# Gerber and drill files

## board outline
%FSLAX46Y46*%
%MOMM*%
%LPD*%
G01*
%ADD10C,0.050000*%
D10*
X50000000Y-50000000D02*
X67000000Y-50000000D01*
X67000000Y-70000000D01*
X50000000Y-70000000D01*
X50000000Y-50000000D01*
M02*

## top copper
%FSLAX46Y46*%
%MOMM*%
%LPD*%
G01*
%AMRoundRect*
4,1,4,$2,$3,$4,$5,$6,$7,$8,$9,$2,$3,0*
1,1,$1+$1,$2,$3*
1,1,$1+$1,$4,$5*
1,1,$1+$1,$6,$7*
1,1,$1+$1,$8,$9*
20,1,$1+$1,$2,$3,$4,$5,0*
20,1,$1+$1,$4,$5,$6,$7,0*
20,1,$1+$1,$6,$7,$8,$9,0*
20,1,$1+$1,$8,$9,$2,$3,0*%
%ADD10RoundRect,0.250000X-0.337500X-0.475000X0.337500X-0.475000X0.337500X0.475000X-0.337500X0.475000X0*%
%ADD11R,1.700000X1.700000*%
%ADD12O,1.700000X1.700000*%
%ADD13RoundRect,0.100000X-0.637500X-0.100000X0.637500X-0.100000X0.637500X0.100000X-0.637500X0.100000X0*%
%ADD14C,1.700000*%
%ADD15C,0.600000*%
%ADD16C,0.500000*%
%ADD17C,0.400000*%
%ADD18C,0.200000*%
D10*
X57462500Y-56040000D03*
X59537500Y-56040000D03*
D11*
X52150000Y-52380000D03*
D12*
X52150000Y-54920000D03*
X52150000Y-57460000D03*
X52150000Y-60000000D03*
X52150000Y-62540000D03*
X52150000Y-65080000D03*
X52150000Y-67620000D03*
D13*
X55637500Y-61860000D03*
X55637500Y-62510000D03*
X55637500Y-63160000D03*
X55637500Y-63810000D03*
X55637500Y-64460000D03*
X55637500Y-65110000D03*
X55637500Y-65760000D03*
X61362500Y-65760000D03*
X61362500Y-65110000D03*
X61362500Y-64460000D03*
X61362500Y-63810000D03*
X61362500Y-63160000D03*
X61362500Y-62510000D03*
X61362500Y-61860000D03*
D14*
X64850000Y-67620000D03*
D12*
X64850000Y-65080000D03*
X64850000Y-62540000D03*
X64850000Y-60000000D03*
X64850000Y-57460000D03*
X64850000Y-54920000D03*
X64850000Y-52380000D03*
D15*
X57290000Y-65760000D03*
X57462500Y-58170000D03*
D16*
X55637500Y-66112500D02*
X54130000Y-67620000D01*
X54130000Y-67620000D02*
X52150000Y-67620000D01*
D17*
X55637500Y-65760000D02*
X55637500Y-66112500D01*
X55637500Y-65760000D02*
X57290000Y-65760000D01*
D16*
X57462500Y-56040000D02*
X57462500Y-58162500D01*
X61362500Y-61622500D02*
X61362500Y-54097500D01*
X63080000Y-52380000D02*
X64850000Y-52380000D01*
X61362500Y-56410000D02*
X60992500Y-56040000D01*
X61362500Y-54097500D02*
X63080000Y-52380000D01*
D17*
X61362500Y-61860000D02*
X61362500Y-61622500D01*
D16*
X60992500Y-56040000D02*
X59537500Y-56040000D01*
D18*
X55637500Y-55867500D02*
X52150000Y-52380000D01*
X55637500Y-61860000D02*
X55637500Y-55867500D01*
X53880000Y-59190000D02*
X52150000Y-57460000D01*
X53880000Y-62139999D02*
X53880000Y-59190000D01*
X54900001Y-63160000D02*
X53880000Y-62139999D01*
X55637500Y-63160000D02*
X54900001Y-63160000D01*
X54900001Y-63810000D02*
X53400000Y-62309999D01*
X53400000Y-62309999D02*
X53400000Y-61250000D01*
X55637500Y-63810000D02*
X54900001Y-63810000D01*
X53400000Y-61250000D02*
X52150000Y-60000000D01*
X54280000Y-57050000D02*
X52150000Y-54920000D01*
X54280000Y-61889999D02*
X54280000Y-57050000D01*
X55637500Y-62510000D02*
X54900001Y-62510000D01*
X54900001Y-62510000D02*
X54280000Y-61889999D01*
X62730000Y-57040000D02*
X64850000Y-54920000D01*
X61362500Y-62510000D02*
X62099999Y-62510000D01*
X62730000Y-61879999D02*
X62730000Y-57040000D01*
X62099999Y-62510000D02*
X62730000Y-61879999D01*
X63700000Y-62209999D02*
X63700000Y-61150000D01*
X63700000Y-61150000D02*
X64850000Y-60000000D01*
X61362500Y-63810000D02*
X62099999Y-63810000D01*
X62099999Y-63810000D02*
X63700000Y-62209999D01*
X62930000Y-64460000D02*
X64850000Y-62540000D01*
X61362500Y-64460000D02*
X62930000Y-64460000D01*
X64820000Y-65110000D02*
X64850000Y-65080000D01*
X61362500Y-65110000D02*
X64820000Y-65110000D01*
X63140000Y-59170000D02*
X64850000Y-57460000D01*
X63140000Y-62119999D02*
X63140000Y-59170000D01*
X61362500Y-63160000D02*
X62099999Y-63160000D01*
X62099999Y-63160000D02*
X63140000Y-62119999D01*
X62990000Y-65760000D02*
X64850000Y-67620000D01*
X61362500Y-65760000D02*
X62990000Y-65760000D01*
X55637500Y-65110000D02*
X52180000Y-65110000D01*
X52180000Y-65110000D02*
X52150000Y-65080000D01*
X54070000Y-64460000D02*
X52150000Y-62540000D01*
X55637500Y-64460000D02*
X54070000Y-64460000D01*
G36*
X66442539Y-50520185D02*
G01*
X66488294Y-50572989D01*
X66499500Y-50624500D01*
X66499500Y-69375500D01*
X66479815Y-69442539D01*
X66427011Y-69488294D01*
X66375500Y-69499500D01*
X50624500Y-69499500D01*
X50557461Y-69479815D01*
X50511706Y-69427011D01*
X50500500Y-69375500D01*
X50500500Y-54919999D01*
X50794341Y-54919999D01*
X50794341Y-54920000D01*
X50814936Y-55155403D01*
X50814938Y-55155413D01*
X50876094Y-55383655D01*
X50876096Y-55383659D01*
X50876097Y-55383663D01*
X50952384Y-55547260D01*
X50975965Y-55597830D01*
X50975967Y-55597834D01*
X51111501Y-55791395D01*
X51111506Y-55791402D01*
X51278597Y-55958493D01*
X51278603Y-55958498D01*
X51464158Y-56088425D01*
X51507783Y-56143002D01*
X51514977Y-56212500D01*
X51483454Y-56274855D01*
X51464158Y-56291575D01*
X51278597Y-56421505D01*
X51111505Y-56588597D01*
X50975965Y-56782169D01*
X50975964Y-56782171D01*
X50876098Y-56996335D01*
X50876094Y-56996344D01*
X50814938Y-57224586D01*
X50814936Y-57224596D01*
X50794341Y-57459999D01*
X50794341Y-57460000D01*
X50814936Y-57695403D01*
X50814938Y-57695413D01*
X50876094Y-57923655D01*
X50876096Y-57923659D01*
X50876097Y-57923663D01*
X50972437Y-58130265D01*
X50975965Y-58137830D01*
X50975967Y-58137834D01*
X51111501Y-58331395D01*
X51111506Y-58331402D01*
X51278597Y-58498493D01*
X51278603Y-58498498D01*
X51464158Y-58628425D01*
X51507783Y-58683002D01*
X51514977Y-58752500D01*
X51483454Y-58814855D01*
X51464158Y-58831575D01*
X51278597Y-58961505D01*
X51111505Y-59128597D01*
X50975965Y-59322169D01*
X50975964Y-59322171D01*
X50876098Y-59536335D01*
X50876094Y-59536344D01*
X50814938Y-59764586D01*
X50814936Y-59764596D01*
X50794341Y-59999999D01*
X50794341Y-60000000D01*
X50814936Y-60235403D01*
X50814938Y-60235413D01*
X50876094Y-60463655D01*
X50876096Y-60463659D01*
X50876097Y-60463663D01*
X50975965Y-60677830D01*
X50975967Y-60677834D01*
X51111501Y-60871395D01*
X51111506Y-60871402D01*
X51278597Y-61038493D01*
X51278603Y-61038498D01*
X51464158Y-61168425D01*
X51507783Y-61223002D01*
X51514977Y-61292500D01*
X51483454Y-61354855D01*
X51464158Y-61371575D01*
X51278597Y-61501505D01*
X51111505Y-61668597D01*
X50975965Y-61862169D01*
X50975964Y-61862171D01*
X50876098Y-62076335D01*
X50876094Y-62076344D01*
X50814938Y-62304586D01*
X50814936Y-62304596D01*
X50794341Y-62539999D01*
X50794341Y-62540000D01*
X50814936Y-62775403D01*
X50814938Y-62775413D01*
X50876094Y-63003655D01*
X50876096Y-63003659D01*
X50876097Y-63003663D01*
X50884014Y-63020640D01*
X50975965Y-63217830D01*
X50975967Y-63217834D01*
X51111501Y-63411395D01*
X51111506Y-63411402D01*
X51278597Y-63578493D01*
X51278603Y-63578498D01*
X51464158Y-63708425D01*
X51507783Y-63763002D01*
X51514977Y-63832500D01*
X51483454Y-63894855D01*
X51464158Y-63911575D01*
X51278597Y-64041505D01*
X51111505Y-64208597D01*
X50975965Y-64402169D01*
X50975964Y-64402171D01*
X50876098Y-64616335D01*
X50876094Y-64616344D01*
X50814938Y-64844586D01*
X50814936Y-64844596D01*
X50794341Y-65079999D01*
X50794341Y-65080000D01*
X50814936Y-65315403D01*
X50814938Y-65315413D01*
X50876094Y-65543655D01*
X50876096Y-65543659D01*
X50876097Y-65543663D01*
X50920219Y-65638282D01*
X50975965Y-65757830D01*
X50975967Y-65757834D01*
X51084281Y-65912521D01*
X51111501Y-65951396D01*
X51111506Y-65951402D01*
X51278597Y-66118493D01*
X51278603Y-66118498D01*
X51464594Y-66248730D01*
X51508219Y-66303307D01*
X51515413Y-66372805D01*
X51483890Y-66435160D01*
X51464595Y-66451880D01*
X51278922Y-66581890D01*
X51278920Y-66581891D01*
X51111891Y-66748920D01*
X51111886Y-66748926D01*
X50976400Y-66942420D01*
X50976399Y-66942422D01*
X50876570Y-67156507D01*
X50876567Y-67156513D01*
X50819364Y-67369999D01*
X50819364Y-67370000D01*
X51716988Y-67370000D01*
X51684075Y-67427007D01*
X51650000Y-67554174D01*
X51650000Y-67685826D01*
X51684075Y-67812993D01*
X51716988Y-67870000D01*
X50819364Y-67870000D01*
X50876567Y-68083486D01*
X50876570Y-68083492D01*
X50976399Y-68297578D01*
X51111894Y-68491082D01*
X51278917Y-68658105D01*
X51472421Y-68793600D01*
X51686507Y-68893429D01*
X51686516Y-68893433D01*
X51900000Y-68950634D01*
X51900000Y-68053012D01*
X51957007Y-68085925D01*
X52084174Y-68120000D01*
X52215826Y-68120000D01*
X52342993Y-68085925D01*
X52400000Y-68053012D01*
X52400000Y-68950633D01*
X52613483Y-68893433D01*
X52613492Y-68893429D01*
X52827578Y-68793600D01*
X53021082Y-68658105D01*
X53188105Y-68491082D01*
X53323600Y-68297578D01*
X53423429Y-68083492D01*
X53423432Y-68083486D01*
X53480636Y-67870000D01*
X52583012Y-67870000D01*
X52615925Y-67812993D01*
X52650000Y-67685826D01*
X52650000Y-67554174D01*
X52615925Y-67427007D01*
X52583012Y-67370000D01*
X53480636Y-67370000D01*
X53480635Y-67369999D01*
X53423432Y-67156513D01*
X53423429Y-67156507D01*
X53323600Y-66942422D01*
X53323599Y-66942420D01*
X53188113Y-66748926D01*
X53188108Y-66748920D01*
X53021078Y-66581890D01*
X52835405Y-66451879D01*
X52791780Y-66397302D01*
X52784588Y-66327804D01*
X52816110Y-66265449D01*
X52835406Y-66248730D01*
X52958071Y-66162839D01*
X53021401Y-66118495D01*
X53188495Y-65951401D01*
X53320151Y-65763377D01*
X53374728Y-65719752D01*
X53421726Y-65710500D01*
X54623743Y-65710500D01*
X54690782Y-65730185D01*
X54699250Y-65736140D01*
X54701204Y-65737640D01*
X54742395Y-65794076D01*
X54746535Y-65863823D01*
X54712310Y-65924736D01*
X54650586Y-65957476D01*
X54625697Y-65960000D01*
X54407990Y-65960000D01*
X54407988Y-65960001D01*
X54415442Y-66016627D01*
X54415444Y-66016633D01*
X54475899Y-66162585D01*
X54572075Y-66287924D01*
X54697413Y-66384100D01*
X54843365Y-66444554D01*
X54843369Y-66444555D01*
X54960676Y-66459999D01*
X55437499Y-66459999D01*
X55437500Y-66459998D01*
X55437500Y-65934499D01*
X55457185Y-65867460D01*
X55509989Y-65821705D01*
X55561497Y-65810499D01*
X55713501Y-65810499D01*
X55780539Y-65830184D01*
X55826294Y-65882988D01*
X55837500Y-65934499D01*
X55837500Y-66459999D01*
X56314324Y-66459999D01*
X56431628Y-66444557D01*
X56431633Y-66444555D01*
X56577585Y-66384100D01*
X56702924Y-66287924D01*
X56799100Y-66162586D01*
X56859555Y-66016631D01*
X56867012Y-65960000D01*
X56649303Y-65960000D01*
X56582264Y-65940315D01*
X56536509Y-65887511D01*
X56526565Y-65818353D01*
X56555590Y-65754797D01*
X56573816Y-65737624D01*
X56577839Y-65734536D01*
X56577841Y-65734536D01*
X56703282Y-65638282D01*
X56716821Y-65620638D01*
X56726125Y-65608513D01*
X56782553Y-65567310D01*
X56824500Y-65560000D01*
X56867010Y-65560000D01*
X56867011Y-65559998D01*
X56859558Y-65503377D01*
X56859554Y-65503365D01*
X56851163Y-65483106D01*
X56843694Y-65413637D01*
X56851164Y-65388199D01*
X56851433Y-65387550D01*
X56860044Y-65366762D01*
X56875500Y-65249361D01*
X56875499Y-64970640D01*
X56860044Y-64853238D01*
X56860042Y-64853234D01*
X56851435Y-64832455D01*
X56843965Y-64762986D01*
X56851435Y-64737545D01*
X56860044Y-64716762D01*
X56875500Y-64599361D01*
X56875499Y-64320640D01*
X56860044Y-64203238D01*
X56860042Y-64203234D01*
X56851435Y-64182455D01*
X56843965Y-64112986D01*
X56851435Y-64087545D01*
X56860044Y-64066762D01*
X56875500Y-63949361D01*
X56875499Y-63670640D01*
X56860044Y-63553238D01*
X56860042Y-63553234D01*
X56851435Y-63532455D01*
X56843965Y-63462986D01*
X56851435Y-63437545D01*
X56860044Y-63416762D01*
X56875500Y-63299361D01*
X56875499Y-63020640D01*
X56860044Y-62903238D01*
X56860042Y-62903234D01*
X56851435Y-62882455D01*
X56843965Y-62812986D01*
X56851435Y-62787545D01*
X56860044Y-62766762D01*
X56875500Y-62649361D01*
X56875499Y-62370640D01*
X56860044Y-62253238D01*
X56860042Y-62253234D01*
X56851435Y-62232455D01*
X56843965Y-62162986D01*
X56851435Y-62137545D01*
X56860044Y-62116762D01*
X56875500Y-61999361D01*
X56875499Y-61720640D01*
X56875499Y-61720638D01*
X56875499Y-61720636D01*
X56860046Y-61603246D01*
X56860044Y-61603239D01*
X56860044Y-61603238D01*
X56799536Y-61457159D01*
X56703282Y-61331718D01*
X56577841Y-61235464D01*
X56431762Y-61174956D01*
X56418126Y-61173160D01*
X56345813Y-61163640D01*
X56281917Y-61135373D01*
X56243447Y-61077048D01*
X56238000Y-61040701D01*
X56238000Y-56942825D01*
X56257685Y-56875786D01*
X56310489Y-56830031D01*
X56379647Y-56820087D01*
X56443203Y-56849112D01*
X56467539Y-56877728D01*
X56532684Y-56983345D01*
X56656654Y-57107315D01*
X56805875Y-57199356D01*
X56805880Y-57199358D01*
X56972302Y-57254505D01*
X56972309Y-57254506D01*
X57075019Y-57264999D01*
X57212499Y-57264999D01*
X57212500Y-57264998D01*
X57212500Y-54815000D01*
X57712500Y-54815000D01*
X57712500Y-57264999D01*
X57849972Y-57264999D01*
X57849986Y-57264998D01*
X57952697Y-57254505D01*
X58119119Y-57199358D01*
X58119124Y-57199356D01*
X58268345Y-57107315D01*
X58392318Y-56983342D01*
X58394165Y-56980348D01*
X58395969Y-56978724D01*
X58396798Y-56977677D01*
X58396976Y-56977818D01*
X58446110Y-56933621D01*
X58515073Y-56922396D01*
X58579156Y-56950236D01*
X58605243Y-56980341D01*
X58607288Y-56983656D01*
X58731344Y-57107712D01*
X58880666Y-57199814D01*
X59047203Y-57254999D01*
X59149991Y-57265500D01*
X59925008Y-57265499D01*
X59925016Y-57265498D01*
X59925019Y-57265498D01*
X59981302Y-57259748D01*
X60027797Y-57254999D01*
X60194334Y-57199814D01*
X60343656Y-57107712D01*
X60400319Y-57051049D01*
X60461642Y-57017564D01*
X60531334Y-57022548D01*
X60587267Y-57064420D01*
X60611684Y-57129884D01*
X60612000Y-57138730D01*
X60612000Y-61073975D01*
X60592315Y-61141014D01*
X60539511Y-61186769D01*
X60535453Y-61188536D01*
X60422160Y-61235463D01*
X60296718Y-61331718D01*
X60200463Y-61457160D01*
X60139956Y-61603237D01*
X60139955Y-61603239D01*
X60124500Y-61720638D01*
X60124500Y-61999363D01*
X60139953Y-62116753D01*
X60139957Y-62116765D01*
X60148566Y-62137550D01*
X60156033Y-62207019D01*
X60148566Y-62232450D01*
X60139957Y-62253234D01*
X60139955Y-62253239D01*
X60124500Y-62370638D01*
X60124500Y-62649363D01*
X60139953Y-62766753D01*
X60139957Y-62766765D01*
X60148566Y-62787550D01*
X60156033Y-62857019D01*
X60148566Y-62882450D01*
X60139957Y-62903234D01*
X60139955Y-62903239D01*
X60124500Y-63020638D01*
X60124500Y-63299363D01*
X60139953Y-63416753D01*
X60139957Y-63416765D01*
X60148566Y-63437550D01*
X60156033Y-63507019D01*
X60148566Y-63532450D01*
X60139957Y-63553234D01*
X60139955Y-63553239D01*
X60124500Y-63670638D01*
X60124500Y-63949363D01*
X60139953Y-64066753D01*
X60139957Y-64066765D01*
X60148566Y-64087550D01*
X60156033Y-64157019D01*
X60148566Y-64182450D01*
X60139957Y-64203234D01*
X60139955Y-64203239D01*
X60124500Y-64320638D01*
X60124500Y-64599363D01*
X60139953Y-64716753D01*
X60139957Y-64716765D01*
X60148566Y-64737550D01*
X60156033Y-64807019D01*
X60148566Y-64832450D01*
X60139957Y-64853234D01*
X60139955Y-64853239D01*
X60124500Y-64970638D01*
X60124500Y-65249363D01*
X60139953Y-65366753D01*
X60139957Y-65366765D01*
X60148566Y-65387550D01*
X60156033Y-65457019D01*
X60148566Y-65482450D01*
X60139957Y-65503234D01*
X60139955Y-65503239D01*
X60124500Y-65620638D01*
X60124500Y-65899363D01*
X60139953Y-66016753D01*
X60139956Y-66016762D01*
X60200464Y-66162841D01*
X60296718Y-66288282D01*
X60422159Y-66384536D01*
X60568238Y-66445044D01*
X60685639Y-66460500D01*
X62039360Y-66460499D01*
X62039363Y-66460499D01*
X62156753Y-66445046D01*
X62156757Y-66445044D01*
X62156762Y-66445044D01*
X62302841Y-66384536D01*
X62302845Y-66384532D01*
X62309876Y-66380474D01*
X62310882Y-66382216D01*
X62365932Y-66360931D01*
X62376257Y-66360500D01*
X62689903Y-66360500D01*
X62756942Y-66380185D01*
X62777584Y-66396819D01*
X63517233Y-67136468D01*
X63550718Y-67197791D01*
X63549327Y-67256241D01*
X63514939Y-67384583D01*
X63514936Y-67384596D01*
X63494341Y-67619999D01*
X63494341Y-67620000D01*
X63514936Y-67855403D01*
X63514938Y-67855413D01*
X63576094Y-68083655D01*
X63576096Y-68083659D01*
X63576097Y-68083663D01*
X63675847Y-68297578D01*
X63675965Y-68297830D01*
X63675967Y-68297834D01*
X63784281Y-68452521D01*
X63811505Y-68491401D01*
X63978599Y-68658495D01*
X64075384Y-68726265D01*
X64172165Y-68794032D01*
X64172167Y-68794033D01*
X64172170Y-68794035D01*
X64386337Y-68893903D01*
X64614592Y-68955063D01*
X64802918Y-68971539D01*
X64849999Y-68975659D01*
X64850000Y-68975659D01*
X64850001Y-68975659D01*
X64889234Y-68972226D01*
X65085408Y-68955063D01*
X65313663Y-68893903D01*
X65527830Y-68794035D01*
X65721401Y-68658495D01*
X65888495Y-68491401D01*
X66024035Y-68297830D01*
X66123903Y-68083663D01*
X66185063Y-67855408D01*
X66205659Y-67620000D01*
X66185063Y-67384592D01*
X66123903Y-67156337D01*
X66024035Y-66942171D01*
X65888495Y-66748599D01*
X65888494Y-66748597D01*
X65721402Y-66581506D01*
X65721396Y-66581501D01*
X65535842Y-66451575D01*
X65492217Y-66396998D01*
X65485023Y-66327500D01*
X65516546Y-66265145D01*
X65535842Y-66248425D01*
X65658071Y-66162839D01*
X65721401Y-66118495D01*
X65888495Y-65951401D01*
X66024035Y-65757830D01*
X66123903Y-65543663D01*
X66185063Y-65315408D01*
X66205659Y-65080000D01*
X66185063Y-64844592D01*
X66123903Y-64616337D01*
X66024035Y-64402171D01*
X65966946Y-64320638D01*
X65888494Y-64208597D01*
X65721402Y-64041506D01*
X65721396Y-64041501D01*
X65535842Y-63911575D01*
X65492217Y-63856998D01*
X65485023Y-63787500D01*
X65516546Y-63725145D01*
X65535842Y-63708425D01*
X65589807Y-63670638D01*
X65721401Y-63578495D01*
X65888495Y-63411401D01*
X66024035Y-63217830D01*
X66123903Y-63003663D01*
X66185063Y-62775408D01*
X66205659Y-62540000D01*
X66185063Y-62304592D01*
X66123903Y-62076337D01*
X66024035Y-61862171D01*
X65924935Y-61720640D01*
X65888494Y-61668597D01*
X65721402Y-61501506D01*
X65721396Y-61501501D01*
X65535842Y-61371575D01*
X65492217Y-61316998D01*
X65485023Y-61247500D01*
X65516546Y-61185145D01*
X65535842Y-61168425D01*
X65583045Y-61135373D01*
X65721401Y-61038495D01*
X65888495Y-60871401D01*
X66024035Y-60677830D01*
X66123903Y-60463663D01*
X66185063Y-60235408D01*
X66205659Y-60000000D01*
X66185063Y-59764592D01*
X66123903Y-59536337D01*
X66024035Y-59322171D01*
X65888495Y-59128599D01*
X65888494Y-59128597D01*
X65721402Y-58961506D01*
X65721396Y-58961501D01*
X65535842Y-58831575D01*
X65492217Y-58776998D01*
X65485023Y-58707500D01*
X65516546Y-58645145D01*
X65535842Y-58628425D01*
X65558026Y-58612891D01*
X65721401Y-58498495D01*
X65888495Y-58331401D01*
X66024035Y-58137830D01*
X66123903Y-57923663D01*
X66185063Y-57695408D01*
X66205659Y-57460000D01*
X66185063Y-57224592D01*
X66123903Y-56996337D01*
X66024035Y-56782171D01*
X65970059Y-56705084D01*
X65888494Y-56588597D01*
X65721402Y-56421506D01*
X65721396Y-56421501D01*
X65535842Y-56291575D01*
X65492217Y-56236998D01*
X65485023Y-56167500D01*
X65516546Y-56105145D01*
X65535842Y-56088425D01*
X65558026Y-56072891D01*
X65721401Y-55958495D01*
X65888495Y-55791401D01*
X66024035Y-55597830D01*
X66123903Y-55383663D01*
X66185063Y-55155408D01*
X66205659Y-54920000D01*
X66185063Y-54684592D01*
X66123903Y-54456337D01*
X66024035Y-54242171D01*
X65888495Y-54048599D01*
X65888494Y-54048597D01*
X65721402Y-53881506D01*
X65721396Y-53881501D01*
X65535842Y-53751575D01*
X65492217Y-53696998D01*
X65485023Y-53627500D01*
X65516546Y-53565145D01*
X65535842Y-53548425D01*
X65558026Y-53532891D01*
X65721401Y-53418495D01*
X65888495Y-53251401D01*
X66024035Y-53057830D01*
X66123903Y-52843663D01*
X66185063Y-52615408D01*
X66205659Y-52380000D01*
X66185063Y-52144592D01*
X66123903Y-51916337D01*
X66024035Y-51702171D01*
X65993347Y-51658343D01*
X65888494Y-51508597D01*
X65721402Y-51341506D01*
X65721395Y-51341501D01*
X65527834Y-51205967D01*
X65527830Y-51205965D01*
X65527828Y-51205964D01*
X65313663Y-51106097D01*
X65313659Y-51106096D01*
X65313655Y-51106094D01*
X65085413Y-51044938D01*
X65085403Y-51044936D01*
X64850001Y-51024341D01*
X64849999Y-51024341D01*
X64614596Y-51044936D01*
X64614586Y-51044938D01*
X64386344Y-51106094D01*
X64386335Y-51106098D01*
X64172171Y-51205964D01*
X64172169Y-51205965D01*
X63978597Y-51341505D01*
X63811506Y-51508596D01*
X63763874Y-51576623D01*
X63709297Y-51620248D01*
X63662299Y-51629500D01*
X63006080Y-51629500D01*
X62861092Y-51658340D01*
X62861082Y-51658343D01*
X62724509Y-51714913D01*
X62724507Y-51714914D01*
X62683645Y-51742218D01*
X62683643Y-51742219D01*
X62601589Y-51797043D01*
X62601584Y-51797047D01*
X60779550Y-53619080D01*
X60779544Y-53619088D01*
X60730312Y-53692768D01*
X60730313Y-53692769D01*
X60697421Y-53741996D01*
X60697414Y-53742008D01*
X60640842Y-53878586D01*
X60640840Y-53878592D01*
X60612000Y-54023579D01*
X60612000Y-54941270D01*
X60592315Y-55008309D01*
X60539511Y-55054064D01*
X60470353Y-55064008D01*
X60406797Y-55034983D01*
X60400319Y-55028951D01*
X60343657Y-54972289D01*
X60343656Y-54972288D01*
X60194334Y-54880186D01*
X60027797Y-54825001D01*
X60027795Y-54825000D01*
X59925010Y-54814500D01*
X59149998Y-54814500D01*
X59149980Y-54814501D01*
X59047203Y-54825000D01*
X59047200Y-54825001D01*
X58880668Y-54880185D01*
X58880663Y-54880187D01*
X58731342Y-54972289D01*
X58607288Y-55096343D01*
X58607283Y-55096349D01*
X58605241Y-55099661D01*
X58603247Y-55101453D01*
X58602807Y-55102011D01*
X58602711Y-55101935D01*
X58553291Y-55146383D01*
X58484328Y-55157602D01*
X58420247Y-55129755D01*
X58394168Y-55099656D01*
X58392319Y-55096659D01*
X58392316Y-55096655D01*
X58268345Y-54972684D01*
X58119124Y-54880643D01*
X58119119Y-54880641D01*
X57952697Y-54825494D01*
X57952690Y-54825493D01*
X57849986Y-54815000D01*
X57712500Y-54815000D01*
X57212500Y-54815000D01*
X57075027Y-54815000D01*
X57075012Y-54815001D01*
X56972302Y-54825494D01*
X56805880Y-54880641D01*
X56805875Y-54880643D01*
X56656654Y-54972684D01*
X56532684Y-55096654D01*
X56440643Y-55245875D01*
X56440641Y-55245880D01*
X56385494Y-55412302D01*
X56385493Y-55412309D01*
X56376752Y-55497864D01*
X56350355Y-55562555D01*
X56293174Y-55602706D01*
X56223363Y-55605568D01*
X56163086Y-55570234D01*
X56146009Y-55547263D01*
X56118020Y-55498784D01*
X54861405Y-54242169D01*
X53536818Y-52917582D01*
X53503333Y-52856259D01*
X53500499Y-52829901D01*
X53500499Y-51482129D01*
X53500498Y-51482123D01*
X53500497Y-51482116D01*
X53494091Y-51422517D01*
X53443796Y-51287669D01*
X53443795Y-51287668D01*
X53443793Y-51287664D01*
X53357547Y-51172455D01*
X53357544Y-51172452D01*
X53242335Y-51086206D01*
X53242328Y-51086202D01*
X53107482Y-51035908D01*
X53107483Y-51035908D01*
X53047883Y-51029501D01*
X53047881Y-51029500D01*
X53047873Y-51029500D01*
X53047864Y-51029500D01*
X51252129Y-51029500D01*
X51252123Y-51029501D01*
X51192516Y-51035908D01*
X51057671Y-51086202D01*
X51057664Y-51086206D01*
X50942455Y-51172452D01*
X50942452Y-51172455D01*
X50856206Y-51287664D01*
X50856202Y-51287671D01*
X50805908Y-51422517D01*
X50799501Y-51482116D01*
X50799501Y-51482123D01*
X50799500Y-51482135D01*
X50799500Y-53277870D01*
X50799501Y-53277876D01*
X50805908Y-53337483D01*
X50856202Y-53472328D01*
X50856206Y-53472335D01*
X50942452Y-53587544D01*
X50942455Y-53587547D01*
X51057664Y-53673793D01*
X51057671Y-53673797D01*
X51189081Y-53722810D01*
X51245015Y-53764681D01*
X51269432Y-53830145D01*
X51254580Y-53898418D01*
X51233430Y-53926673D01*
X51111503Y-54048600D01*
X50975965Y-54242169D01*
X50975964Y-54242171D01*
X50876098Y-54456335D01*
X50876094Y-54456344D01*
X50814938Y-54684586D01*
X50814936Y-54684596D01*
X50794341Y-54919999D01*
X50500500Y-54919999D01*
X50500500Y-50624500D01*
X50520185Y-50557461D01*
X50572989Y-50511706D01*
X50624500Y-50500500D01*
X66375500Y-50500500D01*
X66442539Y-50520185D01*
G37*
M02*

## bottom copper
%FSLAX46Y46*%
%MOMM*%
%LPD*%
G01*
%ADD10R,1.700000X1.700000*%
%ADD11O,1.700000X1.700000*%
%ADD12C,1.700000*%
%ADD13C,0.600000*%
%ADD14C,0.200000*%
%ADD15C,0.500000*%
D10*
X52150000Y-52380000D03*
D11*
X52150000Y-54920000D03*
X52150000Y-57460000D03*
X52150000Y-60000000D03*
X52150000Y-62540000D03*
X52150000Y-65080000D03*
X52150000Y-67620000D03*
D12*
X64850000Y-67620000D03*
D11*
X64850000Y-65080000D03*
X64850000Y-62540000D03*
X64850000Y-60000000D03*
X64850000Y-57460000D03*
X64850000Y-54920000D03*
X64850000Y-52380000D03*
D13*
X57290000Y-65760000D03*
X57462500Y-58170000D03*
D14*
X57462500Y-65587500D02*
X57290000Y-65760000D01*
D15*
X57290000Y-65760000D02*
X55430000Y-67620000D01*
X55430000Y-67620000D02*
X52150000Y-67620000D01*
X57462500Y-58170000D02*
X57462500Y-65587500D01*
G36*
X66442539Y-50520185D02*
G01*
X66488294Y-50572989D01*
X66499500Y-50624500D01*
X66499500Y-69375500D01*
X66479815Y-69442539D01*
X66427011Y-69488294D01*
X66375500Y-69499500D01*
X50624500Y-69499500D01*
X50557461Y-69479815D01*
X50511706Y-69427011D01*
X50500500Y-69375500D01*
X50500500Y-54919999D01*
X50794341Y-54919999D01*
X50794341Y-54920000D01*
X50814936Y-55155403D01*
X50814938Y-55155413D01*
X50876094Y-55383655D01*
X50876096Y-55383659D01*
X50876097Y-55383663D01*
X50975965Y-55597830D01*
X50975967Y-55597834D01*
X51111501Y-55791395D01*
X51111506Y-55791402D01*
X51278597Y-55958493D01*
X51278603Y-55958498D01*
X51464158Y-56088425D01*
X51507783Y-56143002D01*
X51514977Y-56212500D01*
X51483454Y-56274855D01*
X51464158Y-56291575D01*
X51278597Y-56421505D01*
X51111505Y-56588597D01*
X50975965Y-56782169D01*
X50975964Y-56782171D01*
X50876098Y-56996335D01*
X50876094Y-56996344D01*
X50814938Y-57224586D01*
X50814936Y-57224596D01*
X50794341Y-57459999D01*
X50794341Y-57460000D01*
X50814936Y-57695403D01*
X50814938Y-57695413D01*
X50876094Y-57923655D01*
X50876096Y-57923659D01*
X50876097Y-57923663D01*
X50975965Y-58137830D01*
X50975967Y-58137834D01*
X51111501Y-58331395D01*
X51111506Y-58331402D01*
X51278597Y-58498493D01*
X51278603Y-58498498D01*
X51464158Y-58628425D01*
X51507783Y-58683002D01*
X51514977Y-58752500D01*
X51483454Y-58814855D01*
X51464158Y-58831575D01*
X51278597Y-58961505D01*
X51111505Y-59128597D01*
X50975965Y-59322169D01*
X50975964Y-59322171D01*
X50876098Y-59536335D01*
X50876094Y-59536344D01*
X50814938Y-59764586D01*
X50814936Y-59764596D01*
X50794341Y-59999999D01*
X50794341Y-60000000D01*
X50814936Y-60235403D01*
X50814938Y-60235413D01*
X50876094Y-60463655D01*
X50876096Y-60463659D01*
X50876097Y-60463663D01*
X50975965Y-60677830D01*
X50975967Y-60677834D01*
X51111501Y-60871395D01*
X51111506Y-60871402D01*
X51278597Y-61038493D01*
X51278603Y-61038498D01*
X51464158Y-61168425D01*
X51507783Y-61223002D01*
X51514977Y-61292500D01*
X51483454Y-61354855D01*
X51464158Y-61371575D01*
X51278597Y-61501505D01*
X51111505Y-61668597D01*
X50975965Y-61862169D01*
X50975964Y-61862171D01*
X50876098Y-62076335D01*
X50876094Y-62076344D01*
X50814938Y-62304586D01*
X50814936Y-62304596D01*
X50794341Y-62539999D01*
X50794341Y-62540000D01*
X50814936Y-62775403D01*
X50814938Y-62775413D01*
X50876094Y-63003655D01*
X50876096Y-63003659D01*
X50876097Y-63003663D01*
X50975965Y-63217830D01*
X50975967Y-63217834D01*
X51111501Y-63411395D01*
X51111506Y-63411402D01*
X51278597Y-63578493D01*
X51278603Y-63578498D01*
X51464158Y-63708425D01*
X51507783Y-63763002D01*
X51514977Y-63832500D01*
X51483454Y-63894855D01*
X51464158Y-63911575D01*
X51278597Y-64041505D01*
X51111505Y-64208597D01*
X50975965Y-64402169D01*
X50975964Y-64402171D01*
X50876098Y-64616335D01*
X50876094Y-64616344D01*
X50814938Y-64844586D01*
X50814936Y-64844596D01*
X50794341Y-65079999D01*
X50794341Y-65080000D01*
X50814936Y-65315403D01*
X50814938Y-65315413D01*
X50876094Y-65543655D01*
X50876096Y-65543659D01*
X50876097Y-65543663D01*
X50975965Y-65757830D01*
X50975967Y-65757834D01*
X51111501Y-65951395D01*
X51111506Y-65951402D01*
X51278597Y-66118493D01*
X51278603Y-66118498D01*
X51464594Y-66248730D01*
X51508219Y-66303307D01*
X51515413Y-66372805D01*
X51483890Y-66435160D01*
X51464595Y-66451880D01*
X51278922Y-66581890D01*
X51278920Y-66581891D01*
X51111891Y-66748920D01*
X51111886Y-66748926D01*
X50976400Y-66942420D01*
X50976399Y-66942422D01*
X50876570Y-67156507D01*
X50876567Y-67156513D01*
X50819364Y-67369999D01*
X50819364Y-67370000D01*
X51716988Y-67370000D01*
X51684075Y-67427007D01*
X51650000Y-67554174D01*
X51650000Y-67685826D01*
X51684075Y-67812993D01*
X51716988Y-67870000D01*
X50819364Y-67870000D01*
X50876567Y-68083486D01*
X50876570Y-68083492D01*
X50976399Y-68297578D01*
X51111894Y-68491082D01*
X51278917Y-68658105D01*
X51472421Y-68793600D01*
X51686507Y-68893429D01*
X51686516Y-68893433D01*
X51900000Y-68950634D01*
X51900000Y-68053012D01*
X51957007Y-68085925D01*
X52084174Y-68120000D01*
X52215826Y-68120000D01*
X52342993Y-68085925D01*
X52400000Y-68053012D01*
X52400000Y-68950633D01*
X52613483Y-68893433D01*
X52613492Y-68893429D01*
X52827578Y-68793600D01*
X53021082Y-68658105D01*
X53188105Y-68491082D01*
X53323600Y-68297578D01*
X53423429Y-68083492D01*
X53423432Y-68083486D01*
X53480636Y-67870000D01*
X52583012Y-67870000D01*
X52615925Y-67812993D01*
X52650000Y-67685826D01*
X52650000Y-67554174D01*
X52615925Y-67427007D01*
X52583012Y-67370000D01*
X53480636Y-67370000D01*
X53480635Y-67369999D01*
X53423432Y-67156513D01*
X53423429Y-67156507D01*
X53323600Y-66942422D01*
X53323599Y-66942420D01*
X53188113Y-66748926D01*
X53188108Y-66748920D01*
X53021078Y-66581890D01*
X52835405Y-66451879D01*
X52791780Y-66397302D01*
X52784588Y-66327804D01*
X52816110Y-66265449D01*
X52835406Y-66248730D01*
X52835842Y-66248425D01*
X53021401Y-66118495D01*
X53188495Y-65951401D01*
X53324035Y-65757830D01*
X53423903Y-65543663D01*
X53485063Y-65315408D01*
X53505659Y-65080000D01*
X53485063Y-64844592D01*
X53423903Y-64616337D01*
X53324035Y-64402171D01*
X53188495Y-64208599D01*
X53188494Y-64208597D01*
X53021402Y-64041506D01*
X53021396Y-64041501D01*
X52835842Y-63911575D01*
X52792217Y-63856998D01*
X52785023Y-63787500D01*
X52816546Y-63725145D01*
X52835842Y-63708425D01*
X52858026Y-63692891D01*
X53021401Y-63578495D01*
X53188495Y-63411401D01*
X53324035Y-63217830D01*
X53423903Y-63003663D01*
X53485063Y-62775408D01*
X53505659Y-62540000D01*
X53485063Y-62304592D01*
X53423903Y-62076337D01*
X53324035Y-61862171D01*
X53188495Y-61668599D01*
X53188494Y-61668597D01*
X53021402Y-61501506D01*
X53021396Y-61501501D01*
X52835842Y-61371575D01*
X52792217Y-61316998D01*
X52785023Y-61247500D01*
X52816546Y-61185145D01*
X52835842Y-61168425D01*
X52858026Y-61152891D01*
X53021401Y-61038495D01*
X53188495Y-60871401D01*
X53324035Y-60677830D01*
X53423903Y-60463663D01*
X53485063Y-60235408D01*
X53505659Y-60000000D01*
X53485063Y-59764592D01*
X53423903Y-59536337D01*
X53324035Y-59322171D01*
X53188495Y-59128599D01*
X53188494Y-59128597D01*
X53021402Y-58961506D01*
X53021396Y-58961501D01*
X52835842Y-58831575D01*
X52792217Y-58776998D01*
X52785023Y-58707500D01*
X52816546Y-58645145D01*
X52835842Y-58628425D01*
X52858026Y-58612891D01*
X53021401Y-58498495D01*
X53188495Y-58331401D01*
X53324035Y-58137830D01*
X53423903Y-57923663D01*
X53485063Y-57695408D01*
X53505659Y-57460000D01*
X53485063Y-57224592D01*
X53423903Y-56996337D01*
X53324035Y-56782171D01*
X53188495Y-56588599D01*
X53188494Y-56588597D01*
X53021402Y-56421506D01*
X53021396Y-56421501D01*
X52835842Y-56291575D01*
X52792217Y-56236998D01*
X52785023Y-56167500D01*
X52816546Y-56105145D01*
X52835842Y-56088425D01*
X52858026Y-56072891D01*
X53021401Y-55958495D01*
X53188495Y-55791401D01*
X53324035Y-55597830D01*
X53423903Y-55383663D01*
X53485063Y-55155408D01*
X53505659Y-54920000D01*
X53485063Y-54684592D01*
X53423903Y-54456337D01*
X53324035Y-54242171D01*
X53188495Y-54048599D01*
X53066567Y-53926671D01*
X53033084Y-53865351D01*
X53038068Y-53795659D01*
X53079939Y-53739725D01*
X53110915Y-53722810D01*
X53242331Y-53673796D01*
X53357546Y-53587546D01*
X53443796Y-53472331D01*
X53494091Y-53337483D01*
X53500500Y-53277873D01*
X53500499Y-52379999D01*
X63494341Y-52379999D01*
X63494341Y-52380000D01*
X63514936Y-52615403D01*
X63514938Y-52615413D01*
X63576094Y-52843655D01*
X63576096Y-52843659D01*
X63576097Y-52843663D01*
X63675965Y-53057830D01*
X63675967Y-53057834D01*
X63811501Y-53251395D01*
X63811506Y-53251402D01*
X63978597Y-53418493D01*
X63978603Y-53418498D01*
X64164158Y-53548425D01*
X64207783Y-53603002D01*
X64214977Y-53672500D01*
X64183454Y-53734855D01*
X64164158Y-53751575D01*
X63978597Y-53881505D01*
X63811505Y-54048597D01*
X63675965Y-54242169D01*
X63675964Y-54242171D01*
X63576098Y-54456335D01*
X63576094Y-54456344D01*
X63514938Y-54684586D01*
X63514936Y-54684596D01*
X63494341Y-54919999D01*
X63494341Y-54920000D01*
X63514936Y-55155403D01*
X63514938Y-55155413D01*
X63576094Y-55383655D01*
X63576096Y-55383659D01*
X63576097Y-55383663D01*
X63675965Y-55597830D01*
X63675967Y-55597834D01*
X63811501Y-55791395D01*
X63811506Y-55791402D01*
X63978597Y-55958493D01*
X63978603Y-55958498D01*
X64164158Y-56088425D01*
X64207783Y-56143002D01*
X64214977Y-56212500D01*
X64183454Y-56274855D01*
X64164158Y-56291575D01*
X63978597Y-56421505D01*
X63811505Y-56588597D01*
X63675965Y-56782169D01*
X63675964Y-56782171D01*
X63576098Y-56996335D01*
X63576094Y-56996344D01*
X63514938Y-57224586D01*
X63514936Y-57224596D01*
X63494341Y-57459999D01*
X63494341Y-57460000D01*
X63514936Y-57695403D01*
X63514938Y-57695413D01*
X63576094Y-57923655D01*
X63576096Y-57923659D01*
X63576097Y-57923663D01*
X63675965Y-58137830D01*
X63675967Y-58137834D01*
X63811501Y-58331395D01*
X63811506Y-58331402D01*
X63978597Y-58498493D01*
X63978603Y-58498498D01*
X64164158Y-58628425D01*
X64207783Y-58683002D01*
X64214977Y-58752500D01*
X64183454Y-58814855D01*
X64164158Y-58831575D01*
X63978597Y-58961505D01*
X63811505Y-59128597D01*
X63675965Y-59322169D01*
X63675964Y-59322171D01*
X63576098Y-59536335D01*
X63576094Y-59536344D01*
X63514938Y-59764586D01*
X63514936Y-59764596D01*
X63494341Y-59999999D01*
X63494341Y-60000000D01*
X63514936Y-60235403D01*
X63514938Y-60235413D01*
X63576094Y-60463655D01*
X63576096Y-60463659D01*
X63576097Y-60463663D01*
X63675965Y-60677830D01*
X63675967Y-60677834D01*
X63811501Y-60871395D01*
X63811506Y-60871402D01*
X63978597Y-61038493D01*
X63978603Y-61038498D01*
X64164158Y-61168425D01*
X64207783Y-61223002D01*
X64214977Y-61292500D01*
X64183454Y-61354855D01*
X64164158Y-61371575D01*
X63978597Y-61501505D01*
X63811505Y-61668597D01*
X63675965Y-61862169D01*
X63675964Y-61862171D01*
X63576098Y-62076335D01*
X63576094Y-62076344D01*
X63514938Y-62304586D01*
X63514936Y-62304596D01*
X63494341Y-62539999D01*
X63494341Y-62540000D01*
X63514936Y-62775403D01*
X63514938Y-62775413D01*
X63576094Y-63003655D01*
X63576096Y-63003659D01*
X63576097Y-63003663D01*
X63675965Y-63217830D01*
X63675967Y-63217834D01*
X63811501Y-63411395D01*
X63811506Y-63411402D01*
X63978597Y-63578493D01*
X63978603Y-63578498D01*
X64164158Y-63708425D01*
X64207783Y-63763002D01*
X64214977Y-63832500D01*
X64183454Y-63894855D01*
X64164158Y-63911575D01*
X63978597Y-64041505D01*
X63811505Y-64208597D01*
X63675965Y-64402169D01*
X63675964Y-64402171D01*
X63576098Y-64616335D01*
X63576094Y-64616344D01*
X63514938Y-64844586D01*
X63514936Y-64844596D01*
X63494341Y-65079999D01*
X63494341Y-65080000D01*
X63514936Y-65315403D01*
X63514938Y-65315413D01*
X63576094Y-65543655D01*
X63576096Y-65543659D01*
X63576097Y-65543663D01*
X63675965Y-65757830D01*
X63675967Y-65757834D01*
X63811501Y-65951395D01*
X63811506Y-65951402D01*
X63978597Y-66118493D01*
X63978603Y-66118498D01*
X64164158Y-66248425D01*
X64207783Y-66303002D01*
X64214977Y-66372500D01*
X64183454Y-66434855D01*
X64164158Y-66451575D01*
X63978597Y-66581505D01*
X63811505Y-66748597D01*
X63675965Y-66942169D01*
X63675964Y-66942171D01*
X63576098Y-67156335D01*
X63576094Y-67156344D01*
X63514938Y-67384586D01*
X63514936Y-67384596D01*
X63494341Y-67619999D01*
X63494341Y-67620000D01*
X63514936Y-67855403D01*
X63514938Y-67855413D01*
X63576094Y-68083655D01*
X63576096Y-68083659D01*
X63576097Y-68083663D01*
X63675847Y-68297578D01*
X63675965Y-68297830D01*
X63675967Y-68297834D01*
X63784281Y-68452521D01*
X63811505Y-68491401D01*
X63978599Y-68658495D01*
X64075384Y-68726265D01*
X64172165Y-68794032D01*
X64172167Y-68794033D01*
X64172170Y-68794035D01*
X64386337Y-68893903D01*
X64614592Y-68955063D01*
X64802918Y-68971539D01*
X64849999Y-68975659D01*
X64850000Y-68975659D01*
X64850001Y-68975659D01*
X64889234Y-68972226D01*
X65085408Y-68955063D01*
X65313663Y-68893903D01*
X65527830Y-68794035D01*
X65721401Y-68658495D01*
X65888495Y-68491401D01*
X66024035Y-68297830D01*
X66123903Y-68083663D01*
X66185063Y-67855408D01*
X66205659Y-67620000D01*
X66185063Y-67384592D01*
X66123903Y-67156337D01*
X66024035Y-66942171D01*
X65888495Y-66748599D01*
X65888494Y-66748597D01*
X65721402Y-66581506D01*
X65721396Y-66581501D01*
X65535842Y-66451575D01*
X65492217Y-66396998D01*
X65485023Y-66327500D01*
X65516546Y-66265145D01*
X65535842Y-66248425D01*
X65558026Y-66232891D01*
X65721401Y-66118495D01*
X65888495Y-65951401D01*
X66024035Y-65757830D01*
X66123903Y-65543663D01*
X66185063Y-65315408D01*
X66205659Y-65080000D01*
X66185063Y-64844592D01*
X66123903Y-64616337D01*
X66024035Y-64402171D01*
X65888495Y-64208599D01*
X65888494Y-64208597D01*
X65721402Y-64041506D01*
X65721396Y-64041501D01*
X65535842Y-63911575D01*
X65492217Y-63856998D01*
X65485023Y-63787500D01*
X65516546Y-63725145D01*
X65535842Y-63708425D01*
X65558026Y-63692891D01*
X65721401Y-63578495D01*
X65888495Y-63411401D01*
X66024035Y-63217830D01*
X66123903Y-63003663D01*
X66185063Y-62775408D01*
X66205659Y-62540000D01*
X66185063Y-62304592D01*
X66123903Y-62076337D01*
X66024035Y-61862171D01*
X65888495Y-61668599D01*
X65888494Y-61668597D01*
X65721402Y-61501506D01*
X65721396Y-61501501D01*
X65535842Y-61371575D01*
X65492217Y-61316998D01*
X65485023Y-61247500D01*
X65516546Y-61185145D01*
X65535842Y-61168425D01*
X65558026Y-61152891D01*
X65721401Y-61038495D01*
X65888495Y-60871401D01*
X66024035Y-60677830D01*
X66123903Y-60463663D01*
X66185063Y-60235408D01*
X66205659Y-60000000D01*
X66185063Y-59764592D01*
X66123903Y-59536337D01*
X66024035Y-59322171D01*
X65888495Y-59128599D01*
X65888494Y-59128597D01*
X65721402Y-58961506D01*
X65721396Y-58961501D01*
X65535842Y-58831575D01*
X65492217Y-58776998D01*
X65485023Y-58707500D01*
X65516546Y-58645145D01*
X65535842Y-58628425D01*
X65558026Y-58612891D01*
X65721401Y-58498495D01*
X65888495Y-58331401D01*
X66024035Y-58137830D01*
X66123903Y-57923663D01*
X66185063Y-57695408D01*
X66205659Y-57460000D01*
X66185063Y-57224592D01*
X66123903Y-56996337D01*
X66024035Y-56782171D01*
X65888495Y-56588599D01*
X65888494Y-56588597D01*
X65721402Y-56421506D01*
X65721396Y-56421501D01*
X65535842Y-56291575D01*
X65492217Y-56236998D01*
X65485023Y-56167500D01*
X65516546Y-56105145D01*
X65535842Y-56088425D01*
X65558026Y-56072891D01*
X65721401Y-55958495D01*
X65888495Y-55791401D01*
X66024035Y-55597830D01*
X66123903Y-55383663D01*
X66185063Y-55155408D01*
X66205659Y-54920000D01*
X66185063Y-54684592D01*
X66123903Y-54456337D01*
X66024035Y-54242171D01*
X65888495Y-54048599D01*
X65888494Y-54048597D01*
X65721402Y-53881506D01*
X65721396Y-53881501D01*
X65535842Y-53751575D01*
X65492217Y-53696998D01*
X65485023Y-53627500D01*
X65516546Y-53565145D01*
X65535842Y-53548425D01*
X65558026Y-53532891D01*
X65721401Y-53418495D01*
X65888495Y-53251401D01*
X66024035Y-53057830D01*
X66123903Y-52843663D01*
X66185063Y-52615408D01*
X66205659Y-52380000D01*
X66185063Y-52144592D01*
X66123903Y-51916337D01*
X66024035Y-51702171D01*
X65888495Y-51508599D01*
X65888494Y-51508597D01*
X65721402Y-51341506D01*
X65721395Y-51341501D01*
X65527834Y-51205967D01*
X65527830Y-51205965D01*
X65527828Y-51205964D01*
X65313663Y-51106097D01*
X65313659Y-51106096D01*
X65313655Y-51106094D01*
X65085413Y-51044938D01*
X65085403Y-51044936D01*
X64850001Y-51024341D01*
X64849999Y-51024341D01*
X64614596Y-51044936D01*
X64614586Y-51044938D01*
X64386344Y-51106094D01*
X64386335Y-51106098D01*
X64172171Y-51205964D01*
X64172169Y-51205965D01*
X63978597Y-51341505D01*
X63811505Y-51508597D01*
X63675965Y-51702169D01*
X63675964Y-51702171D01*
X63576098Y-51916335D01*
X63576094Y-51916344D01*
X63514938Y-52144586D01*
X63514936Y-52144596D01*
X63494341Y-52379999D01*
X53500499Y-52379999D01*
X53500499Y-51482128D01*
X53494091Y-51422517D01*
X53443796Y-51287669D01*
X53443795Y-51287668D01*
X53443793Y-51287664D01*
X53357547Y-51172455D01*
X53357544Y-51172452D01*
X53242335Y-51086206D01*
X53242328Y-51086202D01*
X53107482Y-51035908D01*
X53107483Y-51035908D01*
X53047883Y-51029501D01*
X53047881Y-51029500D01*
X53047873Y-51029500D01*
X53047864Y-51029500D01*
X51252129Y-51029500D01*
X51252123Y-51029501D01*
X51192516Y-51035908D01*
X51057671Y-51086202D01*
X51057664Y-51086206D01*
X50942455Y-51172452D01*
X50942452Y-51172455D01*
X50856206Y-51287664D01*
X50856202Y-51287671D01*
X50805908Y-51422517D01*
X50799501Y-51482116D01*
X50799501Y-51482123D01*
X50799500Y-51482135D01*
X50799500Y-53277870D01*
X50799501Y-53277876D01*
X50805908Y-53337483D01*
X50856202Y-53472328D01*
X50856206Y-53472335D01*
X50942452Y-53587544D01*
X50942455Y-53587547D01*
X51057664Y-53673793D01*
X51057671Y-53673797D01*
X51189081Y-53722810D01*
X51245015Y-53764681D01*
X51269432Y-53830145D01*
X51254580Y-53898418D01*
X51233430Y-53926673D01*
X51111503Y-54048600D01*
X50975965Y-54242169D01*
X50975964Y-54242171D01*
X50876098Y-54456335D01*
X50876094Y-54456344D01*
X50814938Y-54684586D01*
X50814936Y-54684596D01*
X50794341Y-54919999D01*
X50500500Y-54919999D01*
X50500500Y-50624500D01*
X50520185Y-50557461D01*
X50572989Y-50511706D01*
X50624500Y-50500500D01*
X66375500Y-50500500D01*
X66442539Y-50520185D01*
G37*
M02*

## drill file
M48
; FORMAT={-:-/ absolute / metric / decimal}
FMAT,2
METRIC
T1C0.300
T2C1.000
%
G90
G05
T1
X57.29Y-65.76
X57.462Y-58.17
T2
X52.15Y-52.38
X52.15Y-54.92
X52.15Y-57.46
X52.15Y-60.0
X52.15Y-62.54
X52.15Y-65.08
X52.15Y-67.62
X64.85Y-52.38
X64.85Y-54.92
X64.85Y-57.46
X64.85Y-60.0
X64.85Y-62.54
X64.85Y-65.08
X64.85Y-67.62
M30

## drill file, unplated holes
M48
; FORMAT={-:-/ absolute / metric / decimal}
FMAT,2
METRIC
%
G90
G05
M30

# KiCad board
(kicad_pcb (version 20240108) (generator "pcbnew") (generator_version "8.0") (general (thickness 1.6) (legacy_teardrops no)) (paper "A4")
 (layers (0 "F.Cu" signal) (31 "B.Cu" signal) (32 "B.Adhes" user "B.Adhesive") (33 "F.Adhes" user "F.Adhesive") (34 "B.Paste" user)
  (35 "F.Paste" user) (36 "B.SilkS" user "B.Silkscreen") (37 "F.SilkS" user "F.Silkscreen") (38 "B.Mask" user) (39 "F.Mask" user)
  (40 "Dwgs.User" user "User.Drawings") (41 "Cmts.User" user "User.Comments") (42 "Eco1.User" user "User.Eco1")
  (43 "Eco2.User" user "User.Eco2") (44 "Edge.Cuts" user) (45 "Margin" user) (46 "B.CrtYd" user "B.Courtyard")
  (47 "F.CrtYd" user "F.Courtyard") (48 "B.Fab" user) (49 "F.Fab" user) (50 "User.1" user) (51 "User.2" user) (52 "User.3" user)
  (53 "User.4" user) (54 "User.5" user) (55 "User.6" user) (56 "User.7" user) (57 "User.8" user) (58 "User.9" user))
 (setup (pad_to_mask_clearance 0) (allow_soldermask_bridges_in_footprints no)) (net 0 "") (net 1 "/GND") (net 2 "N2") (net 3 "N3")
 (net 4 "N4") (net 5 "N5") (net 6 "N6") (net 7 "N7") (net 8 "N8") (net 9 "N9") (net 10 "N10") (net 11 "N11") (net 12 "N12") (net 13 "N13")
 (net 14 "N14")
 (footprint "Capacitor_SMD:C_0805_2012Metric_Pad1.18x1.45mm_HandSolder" (layer "F.Cu") (at 58.5 56.04)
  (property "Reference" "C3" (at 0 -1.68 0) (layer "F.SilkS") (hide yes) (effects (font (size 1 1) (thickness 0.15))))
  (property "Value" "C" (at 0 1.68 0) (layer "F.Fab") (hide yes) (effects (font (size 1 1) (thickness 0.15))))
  (pad "1" smd roundrect (at -1.0375 0) (size 1.175 1.45) (layers "F.Cu" "F.Paste" "F.Mask") (roundrect_rratio 0.212766) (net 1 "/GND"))
  (pad "2" smd roundrect (at 1.0375 0) (size 1.175 1.45) (layers "F.Cu" "F.Paste" "F.Mask") (roundrect_rratio 0.212766) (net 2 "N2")))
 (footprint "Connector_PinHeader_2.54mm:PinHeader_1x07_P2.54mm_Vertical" (layer "F.Cu") (at 52.15 52.38)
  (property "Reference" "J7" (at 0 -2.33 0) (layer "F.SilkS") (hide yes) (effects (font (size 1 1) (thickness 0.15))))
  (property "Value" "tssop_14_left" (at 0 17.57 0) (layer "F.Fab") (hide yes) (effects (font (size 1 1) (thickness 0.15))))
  (pad "1" thru_hole rect (at 0 0) (size 1.7 1.7) (drill 1) (layers "*.Cu" "*.Mask") (remove_unused_layers no) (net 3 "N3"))
  (pad "2" thru_hole oval (at 0 2.54) (size 1.7 1.7) (drill 1) (layers "*.Cu" "*.Mask") (remove_unused_layers no) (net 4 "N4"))
  (pad "3" thru_hole oval (at 0 5.08) (size 1.7 1.7) (drill 1) (layers "*.Cu" "*.Mask") (remove_unused_layers no) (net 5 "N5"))
  (pad "4" thru_hole oval (at 0 7.62) (size 1.7 1.7) (drill 1) (layers "*.Cu" "*.Mask") (remove_unused_layers no) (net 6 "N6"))
  (pad "5" thru_hole oval (at 0 10.16) (size 1.7 1.7) (drill 1) (layers "*.Cu" "*.Mask") (remove_unused_layers no) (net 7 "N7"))
  (pad "6" thru_hole oval (at 0 12.7) (size 1.7 1.7) (drill 1) (layers "*.Cu" "*.Mask") (remove_unused_layers no) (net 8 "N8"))
  (pad "7" thru_hole oval (at 0 15.24) (size 1.7 1.7) (drill 1) (layers "*.Cu" "*.Mask") (remove_unused_layers no) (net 1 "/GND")))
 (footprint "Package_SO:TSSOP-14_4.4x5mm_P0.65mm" (layer "F.Cu") (at 58.5 63.81)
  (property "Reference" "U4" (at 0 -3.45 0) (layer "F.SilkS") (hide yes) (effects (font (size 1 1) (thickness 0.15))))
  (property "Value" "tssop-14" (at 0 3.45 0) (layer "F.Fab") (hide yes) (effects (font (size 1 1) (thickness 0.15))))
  (pad "1" smd roundrect (at -2.8625 -1.95) (size 1.475 0.4) (layers "F.Cu" "F.Paste" "F.Mask") (roundrect_rratio 0.25) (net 3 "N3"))
  (pad "2" smd roundrect (at -2.8625 -1.3) (size 1.475 0.4) (layers "F.Cu" "F.Paste" "F.Mask") (roundrect_rratio 0.25) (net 4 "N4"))
  (pad "3" smd roundrect (at -2.8625 -0.65) (size 1.475 0.4) (layers "F.Cu" "F.Paste" "F.Mask") (roundrect_rratio 0.25) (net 5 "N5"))
  (pad "4" smd roundrect (at -2.8625 0) (size 1.475 0.4) (layers "F.Cu" "F.Paste" "F.Mask") (roundrect_rratio 0.25) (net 6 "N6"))
  (pad "5" smd roundrect (at -2.8625 0.65) (size 1.475 0.4) (layers "F.Cu" "F.Paste" "F.Mask") (roundrect_rratio 0.25) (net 7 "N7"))
  (pad "6" smd roundrect (at -2.8625 1.3) (size 1.475 0.4) (layers "F.Cu" "F.Paste" "F.Mask") (roundrect_rratio 0.25) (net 8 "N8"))
  (pad "7" smd roundrect (at -2.8625 1.95) (size 1.475 0.4) (layers "F.Cu" "F.Paste" "F.Mask") (roundrect_rratio 0.25) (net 1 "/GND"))
  (pad "8" smd roundrect (at 2.8625 1.95) (size 1.475 0.4) (layers "F.Cu" "F.Paste" "F.Mask") (roundrect_rratio 0.25) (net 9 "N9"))
  (pad "9" smd roundrect (at 2.8625 1.3) (size 1.475 0.4) (layers "F.Cu" "F.Paste" "F.Mask") (roundrect_rratio 0.25) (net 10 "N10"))
  (pad "10" smd roundrect (at 2.8625 0.65) (size 1.475 0.4) (layers "F.Cu" "F.Paste" "F.Mask") (roundrect_rratio 0.25) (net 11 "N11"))
  (pad "11" smd roundrect (at 2.8625 0) (size 1.475 0.4) (layers "F.Cu" "F.Paste" "F.Mask") (roundrect_rratio 0.25) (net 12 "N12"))
  (pad "12" smd roundrect (at 2.8625 -0.65) (size 1.475 0.4) (layers "F.Cu" "F.Paste" "F.Mask") (roundrect_rratio 0.25) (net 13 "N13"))
  (pad "13" smd roundrect (at 2.8625 -1.3) (size 1.475 0.4) (layers "F.Cu" "F.Paste" "F.Mask") (roundrect_rratio 0.25) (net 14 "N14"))
  (pad "14" smd roundrect (at 2.8625 -1.95) (size 1.475 0.4) (layers "F.Cu" "F.Paste" "F.Mask") (roundrect_rratio 0.25) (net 2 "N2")))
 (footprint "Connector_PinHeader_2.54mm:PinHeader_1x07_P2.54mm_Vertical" (layer "F.Cu") (at 64.85 67.62 180)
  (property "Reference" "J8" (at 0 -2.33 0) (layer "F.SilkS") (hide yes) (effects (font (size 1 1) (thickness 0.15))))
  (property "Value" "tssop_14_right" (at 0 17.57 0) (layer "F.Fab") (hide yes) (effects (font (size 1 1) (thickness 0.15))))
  (pad "1" thru_hole circle (at 0 0 180) (size 1.7 1.7) (drill 1) (layers "*.Cu" "*.Mask") (remove_unused_layers no) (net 9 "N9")
   (thermal_bridge_angle 90))
  (pad "2" thru_hole oval (at 0 2.54 180) (size 1.7 1.7) (drill 1) (layers "*.Cu" "*.Mask") (remove_unused_layers no) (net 10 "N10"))
  (pad "3" thru_hole oval (at 0 5.08 180) (size 1.7 1.7) (drill 1) (layers "*.Cu" "*.Mask") (remove_unused_layers no) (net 11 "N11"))
  (pad "4" thru_hole oval (at 0 7.62 180) (size 1.7 1.7) (drill 1) (layers "*.Cu" "*.Mask") (remove_unused_layers no) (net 12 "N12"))
  (pad "5" thru_hole oval (at 0 10.16 180) (size 1.7 1.7) (drill 1) (layers "*.Cu" "*.Mask") (remove_unused_layers no) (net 13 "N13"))
  (pad "6" thru_hole oval (at 0 12.7 180) (size 1.7 1.7) (drill 1) (layers "*.Cu" "*.Mask") (remove_unused_layers no) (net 14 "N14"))
  (pad "7" thru_hole oval (at 0 15.24 180) (size 1.7 1.7) (drill 1) (layers "*.Cu" "*.Mask") (remove_unused_layers no) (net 2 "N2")))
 (gr_rect (start 50 50) (end 67 70) (stroke (width 0.05) (type default)) (fill none) (layer "Edge.Cuts"))
 (segment (start 55.6375 66.1125) (end 54.13 67.62) (width 0.5) (layer "F.Cu") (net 1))
 (segment (start 54.13 67.62) (end 52.15 67.62) (width 0.5) (layer "F.Cu") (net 1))
 (segment (start 55.6375 65.76) (end 55.6375 66.1125) (width 0.4) (layer "F.Cu") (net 1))
 (segment (start 55.6375 65.76) (end 57.29 65.76) (width 0.4) (layer "F.Cu") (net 1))
 (segment (start 57.4625 56.04) (end 57.4625 58.1625) (width 0.5) (layer "F.Cu") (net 1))
 (via (at 57.29 65.76) (size 0.6) (drill 0.3) (layers "F.Cu" "B.Cu") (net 1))
 (via (at 57.4625 58.17) (size 0.6) (drill 0.3) (layers "F.Cu" "B.Cu") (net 1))
 (segment (start 57.4625 65.5875) (end 57.29 65.76) (width 0.2) (layer "B.Cu") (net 1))
 (segment (start 57.29 65.76) (end 55.43 67.62) (width 0.5) (layer "B.Cu") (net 1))
 (segment (start 55.43 67.62) (end 52.15 67.62) (width 0.5) (layer "B.Cu") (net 1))
 (segment (start 57.4625 58.17) (end 57.4625 65.5875) (width 0.5) (layer "B.Cu") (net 1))
 (segment (start 61.3625 61.6225) (end 61.3625 54.0975) (width 0.5) (layer "F.Cu") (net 2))
 (segment (start 63.08 52.38) (end 64.85 52.38) (width 0.5) (layer "F.Cu") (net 2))
 (segment (start 61.3625 56.41) (end 60.9925 56.04) (width 0.5) (layer "F.Cu") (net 2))
 (segment (start 61.3625 54.0975) (end 63.08 52.38) (width 0.5) (layer "F.Cu") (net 2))
 (segment (start 61.3625 61.86) (end 61.3625 61.6225) (width 0.4) (layer "F.Cu") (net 2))
 (segment (start 60.9925 56.04) (end 59.5375 56.04) (width 0.5) (layer "F.Cu") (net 2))
 (segment (start 55.6375 55.8675) (end 52.15 52.38) (width 0.2) (layer "F.Cu") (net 3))
 (segment (start 55.6375 61.86) (end 55.6375 55.8675) (width 0.2) (layer "F.Cu") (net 3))
 (segment (start 53.88 59.19) (end 52.15 57.46) (width 0.2) (layer "F.Cu") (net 5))
 (segment (start 53.88 62.139999) (end 53.88 59.19) (width 0.2) (layer "F.Cu") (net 5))
 (segment (start 54.900001 63.16) (end 53.88 62.139999) (width 0.2) (layer "F.Cu") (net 5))
 (segment (start 55.6375 63.16) (end 54.900001 63.16) (width 0.2) (layer "F.Cu") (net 5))
 (segment (start 54.900001 63.81) (end 53.4 62.309999) (width 0.2) (layer "F.Cu") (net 6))
 (segment (start 53.4 62.309999) (end 53.4 61.25) (width 0.2) (layer "F.Cu") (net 6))
 (segment (start 55.6375 63.81) (end 54.900001 63.81) (width 0.2) (layer "F.Cu") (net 6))
 (segment (start 53.4 61.25) (end 52.15 60) (width 0.2) (layer "F.Cu") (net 6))
 (segment (start 54.28 57.05) (end 52.15 54.92) (width 0.2) (layer "F.Cu") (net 4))
 (segment (start 54.28 61.889999) (end 54.28 57.05) (width 0.2) (layer "F.Cu") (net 4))
 (segment (start 55.6375 62.51) (end 54.900001 62.51) (width 0.2) (layer "F.Cu") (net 4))
 (segment (start 54.900001 62.51) (end 54.28 61.889999) (width 0.2) (layer "F.Cu") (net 4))
 (segment (start 62.73 57.04) (end 64.85 54.92) (width 0.2) (layer "F.Cu") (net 14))
 (segment (start 61.3625 62.51) (end 62.099999 62.51) (width 0.2) (layer "F.Cu") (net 14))
 (segment (start 62.73 61.879999) (end 62.73 57.04) (width 0.2) (layer "F.Cu") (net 14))
 (segment (start 62.099999 62.51) (end 62.73 61.879999) (width 0.2) (layer "F.Cu") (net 14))
 (segment (start 63.7 62.209999) (end 63.7 61.15) (width 0.2) (layer "F.Cu") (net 12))
 (segment (start 63.7 61.15) (end 64.85 60) (width 0.2) (layer "F.Cu") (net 12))
 (segment (start 61.3625 63.81) (end 62.099999 63.81) (width 0.2) (layer "F.Cu") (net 12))
 (segment (start 62.099999 63.81) (end 63.7 62.209999) (width 0.2) (layer "F.Cu") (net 12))
 (segment (start 62.93 64.46) (end 64.85 62.54) (width 0.2) (layer "F.Cu") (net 11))
 (segment (start 61.3625 64.46) (end 62.93 64.46) (width 0.2) (layer "F.Cu") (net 11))
 (segment (start 64.82 65.11) (end 64.85 65.08) (width 0.2) (layer "F.Cu") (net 10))
 (segment (start 61.3625 65.11) (end 64.82 65.11) (width 0.2) (layer "F.Cu") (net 10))
 (segment (start 63.14 59.17) (end 64.85 57.46) (width 0.2) (layer "F.Cu") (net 13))
 (segment (start 63.14 62.119999) (end 63.14 59.17) (width 0.2) (layer "F.Cu") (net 13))
 (segment (start 61.3625 63.16) (end 62.099999 63.16) (width 0.2) (layer "F.Cu") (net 13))
 (segment (start 62.099999 63.16) (end 63.14 62.119999) (width 0.2) (layer "F.Cu") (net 13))
 (segment (start 62.99 65.76) (end 64.85 67.62) (width 0.2) (layer "F.Cu") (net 9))
 (segment (start 61.3625 65.76) (end 62.99 65.76) (width 0.2) (layer "F.Cu") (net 9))
 (segment (start 55.6375 65.11) (end 52.18 65.11) (width 0.2) (layer "F.Cu") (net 8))
 (segment (start 52.18 65.11) (end 52.15 65.08) (width 0.2) (layer "F.Cu") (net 8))
 (segment (start 54.07 64.46) (end 52.15 62.54) (width 0.2) (layer "F.Cu") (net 7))
 (segment (start 55.6375 64.46) (end 54.07 64.46) (width 0.2) (layer "F.Cu") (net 7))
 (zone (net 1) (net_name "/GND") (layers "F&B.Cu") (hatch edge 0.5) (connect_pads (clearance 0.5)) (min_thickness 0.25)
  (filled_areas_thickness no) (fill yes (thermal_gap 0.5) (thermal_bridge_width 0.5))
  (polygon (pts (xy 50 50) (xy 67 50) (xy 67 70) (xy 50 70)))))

